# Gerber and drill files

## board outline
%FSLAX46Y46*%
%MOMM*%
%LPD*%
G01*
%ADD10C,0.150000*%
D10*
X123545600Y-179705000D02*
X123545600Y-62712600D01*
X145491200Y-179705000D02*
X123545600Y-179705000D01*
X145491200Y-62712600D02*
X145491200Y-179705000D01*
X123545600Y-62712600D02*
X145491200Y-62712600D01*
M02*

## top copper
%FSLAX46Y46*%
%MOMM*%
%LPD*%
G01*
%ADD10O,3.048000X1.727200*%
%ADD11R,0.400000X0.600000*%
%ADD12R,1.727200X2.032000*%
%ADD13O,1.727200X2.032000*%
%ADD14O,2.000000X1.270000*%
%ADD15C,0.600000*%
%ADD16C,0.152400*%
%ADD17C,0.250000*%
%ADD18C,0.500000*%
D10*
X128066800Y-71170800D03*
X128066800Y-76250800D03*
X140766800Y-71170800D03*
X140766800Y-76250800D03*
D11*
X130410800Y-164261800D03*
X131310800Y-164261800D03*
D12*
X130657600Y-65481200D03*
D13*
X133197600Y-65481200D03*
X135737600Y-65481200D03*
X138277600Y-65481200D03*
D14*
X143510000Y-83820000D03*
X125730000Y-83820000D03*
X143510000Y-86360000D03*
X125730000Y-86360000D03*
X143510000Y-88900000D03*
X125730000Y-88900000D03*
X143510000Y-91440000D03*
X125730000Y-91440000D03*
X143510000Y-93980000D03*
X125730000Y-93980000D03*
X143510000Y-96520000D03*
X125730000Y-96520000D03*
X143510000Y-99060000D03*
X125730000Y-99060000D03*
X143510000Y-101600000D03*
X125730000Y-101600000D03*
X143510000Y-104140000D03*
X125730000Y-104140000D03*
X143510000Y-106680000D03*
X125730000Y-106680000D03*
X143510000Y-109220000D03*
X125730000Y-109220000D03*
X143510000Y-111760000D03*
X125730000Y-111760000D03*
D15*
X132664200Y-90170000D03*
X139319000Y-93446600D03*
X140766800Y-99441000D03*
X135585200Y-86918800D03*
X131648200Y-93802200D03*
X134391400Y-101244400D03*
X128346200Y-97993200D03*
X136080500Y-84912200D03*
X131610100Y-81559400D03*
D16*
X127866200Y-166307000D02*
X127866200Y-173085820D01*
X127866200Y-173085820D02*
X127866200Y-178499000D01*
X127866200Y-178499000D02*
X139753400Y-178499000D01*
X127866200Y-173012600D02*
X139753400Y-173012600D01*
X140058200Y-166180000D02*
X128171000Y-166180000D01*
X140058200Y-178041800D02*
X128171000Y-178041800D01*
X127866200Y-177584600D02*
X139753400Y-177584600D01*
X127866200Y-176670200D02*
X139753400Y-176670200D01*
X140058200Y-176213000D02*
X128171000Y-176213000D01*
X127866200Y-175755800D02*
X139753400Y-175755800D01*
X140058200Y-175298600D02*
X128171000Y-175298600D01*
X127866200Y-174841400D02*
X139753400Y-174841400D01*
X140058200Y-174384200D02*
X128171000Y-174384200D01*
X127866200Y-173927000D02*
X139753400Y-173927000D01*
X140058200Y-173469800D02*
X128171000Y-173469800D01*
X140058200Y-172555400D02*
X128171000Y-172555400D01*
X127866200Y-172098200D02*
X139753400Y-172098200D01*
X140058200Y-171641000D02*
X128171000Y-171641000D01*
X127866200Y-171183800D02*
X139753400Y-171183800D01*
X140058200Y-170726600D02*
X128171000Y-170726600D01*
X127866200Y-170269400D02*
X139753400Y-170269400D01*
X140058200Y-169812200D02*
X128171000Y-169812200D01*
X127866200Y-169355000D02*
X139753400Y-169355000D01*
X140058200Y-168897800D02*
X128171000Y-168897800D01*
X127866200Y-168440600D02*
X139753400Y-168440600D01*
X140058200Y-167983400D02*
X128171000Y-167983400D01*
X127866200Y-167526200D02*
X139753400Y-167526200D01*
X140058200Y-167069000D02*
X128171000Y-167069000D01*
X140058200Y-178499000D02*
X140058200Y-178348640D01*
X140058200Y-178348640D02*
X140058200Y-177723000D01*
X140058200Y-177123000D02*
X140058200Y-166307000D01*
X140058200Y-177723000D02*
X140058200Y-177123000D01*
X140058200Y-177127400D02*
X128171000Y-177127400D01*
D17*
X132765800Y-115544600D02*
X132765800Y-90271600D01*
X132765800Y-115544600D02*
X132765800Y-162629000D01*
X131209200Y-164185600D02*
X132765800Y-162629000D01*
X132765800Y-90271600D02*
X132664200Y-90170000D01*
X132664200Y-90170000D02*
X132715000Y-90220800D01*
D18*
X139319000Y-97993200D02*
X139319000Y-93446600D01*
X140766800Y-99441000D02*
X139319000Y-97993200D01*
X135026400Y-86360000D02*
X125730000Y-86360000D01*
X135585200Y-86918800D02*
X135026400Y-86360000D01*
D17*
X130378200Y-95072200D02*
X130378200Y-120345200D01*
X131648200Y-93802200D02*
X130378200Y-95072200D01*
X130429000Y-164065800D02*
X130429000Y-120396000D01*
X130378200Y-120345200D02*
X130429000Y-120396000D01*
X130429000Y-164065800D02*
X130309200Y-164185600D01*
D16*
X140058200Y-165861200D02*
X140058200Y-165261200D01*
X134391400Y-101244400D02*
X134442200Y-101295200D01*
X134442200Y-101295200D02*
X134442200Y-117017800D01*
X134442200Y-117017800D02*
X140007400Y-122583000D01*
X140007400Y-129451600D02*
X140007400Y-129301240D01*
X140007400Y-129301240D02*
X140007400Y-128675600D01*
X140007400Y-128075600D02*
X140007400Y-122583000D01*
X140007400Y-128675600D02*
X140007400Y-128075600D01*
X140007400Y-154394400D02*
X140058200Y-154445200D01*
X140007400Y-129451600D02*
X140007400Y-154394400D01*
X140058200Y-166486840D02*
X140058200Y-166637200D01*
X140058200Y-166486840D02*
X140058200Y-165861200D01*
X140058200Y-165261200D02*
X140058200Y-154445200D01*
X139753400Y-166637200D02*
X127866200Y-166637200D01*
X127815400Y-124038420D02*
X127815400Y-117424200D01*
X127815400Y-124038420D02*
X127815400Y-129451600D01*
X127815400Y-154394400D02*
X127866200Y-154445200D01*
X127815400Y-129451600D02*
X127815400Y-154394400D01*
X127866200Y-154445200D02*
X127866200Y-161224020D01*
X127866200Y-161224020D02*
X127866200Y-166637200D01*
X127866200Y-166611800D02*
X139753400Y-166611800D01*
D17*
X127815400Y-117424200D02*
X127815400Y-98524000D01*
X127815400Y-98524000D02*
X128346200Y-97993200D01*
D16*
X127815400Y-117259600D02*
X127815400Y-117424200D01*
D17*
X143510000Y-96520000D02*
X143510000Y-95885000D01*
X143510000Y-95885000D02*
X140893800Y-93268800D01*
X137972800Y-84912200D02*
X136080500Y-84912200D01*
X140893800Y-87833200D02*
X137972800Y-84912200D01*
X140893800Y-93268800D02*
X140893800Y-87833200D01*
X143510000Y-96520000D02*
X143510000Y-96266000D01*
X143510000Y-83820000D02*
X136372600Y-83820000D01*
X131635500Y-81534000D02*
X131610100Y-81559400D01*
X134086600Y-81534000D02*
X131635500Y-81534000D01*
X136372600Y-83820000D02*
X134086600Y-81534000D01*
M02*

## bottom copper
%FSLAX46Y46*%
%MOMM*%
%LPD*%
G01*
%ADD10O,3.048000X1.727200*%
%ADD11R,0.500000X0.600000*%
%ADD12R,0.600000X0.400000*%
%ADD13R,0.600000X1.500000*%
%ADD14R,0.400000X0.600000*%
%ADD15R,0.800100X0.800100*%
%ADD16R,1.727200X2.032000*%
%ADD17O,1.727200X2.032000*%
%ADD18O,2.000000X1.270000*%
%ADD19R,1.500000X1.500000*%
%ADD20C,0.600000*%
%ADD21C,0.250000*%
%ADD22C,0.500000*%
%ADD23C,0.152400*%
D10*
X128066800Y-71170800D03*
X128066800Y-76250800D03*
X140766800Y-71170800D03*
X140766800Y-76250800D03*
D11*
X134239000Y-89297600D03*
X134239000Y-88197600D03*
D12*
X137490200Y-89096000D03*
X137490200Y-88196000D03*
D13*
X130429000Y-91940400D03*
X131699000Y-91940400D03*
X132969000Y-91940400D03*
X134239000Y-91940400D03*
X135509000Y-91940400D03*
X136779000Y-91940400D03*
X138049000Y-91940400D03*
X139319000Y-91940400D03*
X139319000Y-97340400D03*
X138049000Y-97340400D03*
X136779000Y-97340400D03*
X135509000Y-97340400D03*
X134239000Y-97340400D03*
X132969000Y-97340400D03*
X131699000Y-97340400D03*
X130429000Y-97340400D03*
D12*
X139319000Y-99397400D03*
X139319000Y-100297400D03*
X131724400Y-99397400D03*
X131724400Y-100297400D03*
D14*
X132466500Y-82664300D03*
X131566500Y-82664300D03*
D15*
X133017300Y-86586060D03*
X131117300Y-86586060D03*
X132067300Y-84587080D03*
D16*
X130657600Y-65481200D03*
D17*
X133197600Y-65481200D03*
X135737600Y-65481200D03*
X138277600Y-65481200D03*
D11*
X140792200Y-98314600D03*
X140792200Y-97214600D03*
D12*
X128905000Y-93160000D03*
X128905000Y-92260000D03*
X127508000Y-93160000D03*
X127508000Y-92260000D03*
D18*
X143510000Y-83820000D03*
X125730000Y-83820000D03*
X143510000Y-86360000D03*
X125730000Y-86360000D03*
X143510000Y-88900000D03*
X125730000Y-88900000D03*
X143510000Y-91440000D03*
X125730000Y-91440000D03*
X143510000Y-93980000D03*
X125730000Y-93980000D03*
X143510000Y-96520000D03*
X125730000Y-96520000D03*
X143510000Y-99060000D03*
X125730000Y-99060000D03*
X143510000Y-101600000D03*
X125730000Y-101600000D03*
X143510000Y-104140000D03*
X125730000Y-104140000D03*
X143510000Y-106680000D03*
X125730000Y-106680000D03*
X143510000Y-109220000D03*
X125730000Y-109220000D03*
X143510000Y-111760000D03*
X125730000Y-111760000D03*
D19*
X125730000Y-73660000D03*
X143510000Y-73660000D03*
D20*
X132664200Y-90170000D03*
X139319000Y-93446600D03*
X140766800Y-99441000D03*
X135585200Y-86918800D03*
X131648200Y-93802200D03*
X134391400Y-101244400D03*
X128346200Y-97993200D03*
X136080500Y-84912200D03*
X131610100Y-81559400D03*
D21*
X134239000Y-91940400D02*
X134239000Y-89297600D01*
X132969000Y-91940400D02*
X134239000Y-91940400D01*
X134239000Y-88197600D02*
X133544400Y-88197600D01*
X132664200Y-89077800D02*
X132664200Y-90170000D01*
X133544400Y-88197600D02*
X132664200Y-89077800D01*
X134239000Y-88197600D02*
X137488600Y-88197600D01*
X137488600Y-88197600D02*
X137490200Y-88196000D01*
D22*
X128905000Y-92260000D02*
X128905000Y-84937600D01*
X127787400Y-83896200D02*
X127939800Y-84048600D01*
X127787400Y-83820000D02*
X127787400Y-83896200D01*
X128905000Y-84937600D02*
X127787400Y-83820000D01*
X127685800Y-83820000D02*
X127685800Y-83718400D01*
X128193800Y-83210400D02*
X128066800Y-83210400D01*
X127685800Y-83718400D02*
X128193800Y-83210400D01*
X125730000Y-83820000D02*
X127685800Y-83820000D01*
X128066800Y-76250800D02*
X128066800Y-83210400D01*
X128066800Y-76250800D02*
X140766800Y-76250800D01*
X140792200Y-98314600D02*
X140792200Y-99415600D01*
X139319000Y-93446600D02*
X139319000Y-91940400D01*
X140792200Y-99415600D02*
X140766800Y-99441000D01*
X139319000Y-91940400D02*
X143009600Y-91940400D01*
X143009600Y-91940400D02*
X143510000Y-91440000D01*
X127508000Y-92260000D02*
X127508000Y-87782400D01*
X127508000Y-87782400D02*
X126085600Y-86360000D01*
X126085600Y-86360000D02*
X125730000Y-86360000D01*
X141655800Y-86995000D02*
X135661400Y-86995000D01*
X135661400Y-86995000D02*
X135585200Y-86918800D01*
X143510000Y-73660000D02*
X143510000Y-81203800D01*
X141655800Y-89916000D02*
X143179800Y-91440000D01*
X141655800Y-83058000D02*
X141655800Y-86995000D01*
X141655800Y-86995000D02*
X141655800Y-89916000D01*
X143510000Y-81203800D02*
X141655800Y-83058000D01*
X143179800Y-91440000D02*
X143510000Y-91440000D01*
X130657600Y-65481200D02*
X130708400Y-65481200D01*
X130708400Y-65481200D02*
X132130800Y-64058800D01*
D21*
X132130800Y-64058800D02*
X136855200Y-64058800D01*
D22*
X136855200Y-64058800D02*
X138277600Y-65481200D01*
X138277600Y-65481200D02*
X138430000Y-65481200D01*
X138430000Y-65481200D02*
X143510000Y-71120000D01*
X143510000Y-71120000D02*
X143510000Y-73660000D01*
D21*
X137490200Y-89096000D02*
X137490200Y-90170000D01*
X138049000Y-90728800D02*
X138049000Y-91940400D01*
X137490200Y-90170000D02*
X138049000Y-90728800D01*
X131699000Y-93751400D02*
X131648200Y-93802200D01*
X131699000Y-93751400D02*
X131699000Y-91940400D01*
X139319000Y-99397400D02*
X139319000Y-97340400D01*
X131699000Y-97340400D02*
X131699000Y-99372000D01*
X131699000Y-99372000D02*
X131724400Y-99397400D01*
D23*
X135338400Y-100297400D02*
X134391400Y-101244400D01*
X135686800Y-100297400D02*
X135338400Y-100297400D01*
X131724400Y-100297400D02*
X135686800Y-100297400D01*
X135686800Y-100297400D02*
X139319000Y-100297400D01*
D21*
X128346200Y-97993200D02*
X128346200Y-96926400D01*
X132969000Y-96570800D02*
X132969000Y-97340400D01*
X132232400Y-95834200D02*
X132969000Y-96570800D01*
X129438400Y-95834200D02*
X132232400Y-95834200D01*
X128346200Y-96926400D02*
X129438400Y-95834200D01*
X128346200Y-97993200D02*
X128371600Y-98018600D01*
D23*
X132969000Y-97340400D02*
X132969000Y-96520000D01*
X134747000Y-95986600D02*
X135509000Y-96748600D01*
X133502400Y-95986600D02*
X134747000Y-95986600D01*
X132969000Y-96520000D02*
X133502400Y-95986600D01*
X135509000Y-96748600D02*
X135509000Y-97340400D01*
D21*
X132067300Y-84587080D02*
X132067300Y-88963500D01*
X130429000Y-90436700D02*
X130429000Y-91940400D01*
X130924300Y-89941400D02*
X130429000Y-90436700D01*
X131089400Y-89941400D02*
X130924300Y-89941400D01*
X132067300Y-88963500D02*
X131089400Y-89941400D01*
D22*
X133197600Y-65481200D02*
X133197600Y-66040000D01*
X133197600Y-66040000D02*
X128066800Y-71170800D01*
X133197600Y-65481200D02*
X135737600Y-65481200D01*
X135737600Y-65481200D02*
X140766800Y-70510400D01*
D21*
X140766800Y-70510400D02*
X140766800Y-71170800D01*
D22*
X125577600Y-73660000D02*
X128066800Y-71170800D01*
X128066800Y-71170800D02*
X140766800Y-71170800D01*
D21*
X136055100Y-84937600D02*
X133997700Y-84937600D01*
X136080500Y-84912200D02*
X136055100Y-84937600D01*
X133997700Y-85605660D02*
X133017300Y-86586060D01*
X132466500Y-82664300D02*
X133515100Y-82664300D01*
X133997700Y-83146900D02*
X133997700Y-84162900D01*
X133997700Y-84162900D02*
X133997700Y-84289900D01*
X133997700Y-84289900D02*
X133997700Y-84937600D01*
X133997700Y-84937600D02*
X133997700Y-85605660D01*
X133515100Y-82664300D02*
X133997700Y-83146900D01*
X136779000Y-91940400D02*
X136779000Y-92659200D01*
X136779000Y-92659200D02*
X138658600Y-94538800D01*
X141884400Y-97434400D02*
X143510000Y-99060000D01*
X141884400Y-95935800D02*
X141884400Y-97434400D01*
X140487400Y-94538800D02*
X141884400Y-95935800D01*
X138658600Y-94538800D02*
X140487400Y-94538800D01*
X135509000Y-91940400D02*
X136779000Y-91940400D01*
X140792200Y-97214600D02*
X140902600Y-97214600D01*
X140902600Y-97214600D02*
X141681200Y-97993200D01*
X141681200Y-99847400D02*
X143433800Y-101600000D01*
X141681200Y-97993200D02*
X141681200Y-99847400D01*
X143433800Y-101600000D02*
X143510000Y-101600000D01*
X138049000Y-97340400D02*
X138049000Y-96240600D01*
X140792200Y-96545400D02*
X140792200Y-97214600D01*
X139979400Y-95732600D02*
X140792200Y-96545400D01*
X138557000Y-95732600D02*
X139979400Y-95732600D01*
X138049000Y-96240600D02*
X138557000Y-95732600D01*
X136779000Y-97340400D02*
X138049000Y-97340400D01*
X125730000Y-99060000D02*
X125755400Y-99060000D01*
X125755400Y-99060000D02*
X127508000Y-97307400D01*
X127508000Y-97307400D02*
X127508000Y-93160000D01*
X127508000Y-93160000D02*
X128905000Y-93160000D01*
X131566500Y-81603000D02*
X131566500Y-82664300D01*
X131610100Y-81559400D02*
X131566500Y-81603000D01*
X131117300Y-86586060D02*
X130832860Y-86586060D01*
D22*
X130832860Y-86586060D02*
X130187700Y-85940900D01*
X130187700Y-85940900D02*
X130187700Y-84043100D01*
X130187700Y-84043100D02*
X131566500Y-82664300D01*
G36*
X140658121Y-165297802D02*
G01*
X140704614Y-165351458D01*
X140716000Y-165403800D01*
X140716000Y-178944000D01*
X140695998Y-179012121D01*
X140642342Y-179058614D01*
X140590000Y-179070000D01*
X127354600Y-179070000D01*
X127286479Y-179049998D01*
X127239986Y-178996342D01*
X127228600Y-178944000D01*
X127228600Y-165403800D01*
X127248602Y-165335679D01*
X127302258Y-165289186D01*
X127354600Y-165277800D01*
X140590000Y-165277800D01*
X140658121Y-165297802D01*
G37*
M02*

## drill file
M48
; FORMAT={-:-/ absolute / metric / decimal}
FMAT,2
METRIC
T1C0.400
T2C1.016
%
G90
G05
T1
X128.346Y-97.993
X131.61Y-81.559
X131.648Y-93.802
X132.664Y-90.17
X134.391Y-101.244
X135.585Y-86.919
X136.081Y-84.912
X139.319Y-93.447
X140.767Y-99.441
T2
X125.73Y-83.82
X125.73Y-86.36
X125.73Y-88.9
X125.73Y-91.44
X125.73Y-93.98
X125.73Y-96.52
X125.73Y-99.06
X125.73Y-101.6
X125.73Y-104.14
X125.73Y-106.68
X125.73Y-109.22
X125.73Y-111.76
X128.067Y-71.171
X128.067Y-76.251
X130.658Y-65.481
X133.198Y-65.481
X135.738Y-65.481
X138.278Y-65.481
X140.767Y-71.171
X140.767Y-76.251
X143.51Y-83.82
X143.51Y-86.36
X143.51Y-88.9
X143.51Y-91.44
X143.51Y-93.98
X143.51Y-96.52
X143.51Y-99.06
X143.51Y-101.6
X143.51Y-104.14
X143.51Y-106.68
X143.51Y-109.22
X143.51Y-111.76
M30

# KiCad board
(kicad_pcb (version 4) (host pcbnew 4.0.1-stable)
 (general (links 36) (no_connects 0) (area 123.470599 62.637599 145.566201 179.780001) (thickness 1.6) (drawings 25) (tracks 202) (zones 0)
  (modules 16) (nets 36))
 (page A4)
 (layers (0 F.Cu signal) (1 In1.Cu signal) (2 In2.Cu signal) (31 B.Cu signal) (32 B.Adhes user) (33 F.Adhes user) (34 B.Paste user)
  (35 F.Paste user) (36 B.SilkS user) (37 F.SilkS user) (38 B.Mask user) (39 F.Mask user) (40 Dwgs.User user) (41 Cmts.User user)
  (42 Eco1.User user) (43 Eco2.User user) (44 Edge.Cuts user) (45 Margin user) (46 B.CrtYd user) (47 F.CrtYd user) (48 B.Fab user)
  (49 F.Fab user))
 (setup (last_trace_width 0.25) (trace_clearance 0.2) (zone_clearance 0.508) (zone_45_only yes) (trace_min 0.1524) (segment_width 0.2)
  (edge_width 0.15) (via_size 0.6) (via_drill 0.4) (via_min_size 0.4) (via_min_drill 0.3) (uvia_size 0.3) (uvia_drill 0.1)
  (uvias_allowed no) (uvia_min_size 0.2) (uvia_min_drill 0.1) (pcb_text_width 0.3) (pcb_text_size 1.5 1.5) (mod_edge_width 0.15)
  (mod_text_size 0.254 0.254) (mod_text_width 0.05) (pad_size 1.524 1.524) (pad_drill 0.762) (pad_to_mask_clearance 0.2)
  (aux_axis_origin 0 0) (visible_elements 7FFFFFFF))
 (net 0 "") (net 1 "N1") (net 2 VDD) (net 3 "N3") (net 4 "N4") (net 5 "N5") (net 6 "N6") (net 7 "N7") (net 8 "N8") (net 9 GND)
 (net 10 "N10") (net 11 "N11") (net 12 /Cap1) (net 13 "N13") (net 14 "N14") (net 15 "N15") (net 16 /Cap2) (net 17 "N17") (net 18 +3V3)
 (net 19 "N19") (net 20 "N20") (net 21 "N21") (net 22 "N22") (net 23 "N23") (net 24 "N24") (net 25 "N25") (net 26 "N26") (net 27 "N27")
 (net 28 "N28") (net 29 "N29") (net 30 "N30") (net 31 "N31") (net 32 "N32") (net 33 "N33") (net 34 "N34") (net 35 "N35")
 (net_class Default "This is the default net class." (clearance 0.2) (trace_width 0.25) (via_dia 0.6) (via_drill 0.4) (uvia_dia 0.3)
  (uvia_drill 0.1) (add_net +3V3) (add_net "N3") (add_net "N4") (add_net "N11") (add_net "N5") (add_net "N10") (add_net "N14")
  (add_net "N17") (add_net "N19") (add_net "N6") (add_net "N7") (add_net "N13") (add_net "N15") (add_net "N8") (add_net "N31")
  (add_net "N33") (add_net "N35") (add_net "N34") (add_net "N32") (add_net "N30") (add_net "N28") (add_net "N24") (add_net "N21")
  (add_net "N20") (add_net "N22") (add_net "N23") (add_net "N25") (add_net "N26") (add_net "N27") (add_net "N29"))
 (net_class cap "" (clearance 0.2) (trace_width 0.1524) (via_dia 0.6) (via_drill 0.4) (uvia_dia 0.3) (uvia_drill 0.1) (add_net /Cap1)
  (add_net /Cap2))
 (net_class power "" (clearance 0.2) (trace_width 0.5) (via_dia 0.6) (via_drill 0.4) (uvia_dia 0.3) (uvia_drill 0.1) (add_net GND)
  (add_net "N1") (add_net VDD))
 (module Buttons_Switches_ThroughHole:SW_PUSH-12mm (layer B.Cu) (at 134.4168 73.7108 180)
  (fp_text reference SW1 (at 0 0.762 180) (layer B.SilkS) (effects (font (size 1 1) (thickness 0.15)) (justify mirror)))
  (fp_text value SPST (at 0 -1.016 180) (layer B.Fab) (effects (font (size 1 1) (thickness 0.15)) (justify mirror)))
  (pad 1 thru_hole oval (at 6.35 2.54 180) (size 3.048 1.7272) (drill 1.016) (layers *.Cu *.Mask B.SilkS) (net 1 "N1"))
  (pad 2 thru_hole oval (at 6.35 -2.54 180) (size 3.048 1.7272) (drill 1.016) (layers *.Cu *.Mask B.SilkS) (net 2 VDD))
  (pad 1 thru_hole oval (at -6.35 2.54 180) (size 3.048 1.7272) (drill 1.016) (layers *.Cu *.Mask B.SilkS) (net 1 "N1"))
  (pad 2 thru_hole oval (at -6.35 -2.54 180) (size 3.048 1.7272) (drill 1.016) (layers *.Cu *.Mask B.SilkS) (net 2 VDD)))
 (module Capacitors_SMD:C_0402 (layer B.Cu) (at 134.239 88.7476 90)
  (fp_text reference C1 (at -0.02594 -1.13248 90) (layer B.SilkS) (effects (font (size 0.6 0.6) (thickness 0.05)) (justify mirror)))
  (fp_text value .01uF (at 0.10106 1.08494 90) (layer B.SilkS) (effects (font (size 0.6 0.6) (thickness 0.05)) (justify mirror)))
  (pad 1 smd rect (at -0.55 0 90) (size 0.6 0.5) (layers B.Cu B.Paste B.Mask) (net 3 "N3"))
  (pad 2 smd rect (at 0.55 0 90) (size 0.6 0.5) (layers B.Cu B.Paste B.Mask) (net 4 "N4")))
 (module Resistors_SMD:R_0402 (layer B.Cu) (at 137.4902 88.646 90)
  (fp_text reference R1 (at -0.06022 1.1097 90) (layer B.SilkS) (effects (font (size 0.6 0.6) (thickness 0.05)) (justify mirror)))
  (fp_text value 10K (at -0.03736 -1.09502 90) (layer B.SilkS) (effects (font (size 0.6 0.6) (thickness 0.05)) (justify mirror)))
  (pad 1 smd rect (at -0.45 0 90) (size 0.4 0.6) (layers B.Cu B.Paste B.Mask) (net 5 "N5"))
  (pad 2 smd rect (at 0.45 0 90) (size 0.4 0.6) (layers B.Cu B.Paste B.Mask) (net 4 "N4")))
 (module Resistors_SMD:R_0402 (layer F.Cu) (at 130.8608 164.2618)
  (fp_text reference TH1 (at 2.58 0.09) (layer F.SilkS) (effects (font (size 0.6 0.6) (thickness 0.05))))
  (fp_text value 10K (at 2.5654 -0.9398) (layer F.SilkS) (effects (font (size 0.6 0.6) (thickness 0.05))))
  (pad 1 smd rect (at -0.45 0) (size 0.4 0.6) (layers F.Cu F.Paste F.Mask) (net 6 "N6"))
  (pad 2 smd rect (at 0.45 0) (size 0.4 0.6) (layers F.Cu F.Paste F.Mask) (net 4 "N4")))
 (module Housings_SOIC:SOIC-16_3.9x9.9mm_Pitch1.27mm (layer B.Cu) (at 134.874 94.6404 270)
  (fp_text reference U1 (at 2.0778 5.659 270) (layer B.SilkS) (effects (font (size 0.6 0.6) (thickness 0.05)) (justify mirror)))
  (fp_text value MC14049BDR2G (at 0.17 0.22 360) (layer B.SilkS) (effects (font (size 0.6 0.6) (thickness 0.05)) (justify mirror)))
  (pad 1 smd rect (at -2.7 4.445 270) (size 1.5 0.6) (layers B.Cu B.Paste B.Mask) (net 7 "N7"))
  (pad 2 smd rect (at -2.7 3.175 270) (size 1.5 0.6) (layers B.Cu B.Paste B.Mask) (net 6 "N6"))
  (pad 3 smd rect (at -2.7 1.905 270) (size 1.5 0.6) (layers B.Cu B.Paste B.Mask) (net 3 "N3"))
  (pad 4 smd rect (at -2.7 0.635 270) (size 1.5 0.6) (layers B.Cu B.Paste B.Mask) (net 3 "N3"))
  (pad 5 smd rect (at -2.7 -0.635 270) (size 1.5 0.6) (layers B.Cu B.Paste B.Mask) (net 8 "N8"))
  (pad 6 smd rect (at -2.7 -1.905 270) (size 1.5 0.6) (layers B.Cu B.Paste B.Mask) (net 8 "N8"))
  (pad 7 smd rect (at -2.7 -3.175 270) (size 1.5 0.6) (layers B.Cu B.Paste B.Mask) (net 5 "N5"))
  (pad 8 smd rect (at -2.7 -4.445 270) (size 1.5 0.6) (layers B.Cu B.Paste B.Mask) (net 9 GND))
  (pad 9 smd rect (at 2.7 -4.445 270) (size 1.5 0.6) (layers B.Cu B.Paste B.Mask) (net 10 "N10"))
  (pad 10 smd rect (at 2.7 -3.175 270) (size 1.5 0.6) (layers B.Cu B.Paste B.Mask) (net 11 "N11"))
  (pad 11 smd rect (at 2.7 -1.905 270) (size 1.5 0.6) (layers B.Cu B.Paste B.Mask) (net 11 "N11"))
  (pad 12 smd rect (at 2.7 -0.635 270) (size 1.5 0.6) (layers B.Cu B.Paste B.Mask) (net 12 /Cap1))
  (pad 13 smd rect (at 2.7 0.635 270) (size 1.5 0.6) (layers B.Cu B.Paste B.Mask) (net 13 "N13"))
  (pad 14 smd rect (at 2.7 1.905 270) (size 1.5 0.6) (layers B.Cu B.Paste B.Mask) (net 12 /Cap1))
  (pad 15 smd rect (at 2.7 3.175 270) (size 1.5 0.6) (layers B.Cu B.Paste B.Mask) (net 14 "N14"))
  (pad 16 smd rect (at 2.7 4.445 270) (size 1.5 0.6) (layers B.Cu B.Paste B.Mask) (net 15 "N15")))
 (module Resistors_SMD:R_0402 (layer B.Cu) (at 139.319 99.8474 270)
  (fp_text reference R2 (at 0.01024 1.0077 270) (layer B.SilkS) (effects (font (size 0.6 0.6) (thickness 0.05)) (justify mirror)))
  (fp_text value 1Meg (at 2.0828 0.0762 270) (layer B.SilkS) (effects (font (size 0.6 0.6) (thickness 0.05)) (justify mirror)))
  (pad 1 smd rect (at -0.45 0 270) (size 0.4 0.6) (layers B.Cu B.Paste B.Mask) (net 10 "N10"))
  (pad 2 smd rect (at 0.45 0 270) (size 0.4 0.6) (layers B.Cu B.Paste B.Mask) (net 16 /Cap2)))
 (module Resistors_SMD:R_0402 (layer B.Cu) (at 131.7244 99.8474 270)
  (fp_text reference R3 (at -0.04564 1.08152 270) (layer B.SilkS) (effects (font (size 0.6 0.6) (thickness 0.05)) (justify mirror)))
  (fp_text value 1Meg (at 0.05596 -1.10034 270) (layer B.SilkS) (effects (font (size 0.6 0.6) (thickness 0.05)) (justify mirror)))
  (pad 1 smd rect (at -0.45 0 270) (size 0.4 0.6) (layers B.Cu B.Paste B.Mask) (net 14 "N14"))
  (pad 2 smd rect (at 0.45 0 270) (size 0.4 0.6) (layers B.Cu B.Paste B.Mask) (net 16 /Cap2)))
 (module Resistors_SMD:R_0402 (layer B.Cu) (at 132.0165 82.6643 180)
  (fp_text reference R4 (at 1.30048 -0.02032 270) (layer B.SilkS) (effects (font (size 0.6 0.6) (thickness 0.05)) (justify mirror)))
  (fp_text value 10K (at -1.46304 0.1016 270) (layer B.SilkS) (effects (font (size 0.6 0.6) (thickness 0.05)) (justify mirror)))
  (pad 1 smd rect (at -0.45 0 180) (size 0.4 0.6) (layers B.Cu B.Paste B.Mask) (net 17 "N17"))
  (pad 2 smd rect (at 0.45 0 180) (size 0.4 0.6) (layers B.Cu B.Paste B.Mask) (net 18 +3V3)))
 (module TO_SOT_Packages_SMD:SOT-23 (layer B.Cu) (at 132.0673 85.5853 180)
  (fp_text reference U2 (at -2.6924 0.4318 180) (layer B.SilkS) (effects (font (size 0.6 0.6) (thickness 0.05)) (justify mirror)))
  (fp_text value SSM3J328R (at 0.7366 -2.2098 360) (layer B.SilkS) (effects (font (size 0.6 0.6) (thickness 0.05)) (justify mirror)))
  (pad 1 smd rect (at -0.95 -1.00076 180) (size 0.8001 0.8001) (layers B.Cu B.Paste B.Mask) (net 17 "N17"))
  (pad 2 smd rect (at 0.95 -1.00076 180) (size 0.8001 0.8001) (layers B.Cu B.Paste B.Mask) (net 18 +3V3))
  (pad 3 smd rect (at 0 0.99822 180) (size 0.8001 0.8001) (layers B.Cu B.Paste B.Mask) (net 7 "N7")))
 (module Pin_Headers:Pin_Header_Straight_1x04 (layer F.Cu) (at 130.6576 65.4812 90)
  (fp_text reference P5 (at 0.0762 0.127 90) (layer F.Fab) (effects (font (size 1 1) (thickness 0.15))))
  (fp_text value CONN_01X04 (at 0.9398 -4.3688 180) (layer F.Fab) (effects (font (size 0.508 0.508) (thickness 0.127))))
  (pad 1 thru_hole rect (at 0 0 90) (size 2.032 1.7272) (drill 1.016) (layers *.Cu *.Mask F.SilkS) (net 9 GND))
  (pad 2 thru_hole oval (at 0 2.54 90) (size 2.032 1.7272) (drill 1.016) (layers *.Cu *.Mask F.SilkS) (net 1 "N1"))
  (pad 3 thru_hole oval (at 0 5.08 90) (size 2.032 1.7272) (drill 1.016) (layers *.Cu *.Mask F.SilkS) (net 1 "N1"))
  (pad 4 thru_hole oval (at 0 7.62 90) (size 2.032 1.7272) (drill 1.016) (layers *.Cu *.Mask F.SilkS) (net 9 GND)))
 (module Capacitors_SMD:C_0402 (layer B.Cu) (at 140.7922 97.7646 90)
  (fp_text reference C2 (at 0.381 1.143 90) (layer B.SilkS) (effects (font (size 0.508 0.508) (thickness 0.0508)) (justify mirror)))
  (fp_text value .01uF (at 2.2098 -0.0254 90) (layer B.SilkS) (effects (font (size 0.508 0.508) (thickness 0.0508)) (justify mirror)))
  (pad 1 smd rect (at -0.55 0 90) (size 0.6 0.5) (layers B.Cu B.Paste B.Mask) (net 9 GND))
  (pad 2 smd rect (at 0.55 0 90) (size 0.6 0.5) (layers B.Cu B.Paste B.Mask) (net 11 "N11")))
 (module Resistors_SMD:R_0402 (layer B.Cu) (at 128.905 92.71 90)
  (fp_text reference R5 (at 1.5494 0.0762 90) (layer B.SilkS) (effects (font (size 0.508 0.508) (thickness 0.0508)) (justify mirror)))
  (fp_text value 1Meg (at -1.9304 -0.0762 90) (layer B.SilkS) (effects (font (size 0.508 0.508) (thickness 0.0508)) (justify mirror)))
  (pad 1 smd rect (at -0.45 0 90) (size 0.4 0.6) (layers B.Cu B.Paste B.Mask) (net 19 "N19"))
  (pad 2 smd rect (at 0.45 0 90) (size 0.4 0.6) (layers B.Cu B.Paste B.Mask) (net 2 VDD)))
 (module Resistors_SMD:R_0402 (layer B.Cu) (at 127.508 92.71 90)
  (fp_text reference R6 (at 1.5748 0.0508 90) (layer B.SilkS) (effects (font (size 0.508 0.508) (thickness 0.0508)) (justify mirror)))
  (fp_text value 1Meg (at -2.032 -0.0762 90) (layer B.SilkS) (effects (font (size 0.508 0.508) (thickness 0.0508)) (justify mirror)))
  (pad 1 smd rect (at -0.45 0 90) (size 0.4 0.6) (layers B.Cu B.Paste B.Mask) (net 19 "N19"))
  (pad 2 smd rect (at 0.45 0 90) (size 0.4 0.6) (layers B.Cu B.Paste B.Mask) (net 9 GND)))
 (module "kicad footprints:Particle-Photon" (layer F.Cu) (at 134.62 97.79 270)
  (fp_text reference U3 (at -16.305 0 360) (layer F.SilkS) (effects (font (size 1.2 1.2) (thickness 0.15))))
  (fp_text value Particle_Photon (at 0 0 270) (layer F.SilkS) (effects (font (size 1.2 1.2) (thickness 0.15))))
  (pad 24 thru_hole oval (at -13.97 -8.89 270) (size 1.27 2) (drill 1.016) (layers *.Cu *.Mask F.SilkS) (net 18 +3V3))
  (pad 1 thru_hole oval (at -13.97 8.89 270) (size 1.27 2) (drill 1.016) (layers *.Cu *.Mask F.SilkS) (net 2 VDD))
  (pad 23 thru_hole oval (at -11.43 -8.89 270) (size 1.27 2) (drill 1.016) (layers *.Cu *.Mask F.SilkS) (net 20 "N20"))
  (pad 2 thru_hole oval (at -11.43 8.89 270) (size 1.27 2) (drill 1.016) (layers *.Cu *.Mask F.SilkS) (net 9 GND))
  (pad 22 thru_hole oval (at -8.89 -8.89 270) (size 1.27 2) (drill 1.016) (layers *.Cu *.Mask F.SilkS) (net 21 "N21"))
  (pad 3 thru_hole oval (at -8.89 8.89 270) (size 1.27 2) (drill 1.016) (layers *.Cu *.Mask F.SilkS) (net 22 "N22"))
  (pad 21 thru_hole oval (at -6.35 -8.89 270) (size 1.27 2) (drill 1.016) (layers *.Cu *.Mask F.SilkS) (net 9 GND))
  (pad 4 thru_hole oval (at -6.35 8.89 270) (size 1.27 2) (drill 1.016) (layers *.Cu *.Mask F.SilkS) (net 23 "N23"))
  (pad 20 thru_hole oval (at -3.81 -8.89 270) (size 1.27 2) (drill 1.016) (layers *.Cu *.Mask F.SilkS) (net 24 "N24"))
  (pad 5 thru_hole oval (at -3.81 8.89 270) (size 1.27 2) (drill 1.016) (layers *.Cu *.Mask F.SilkS) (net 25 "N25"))
  (pad 19 thru_hole oval (at -1.27 -8.89 270) (size 1.27 2) (drill 1.016) (layers *.Cu *.Mask F.SilkS) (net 17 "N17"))
  (pad 6 thru_hole oval (at -1.27 8.89 270) (size 1.27 2) (drill 1.016) (layers *.Cu *.Mask F.SilkS) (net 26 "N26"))
  (pad 18 thru_hole oval (at 1.27 -8.89 270) (size 1.27 2) (drill 1.016) (layers *.Cu *.Mask F.SilkS) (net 8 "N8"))
  (pad 7 thru_hole oval (at 1.27 8.89 270) (size 1.27 2) (drill 1.016) (layers *.Cu *.Mask F.SilkS) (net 19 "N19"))
  (pad 17 thru_hole oval (at 3.81 -8.89 270) (size 1.27 2) (drill 1.016) (layers *.Cu *.Mask F.SilkS) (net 11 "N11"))
  (pad 8 thru_hole oval (at 3.81 8.89 270) (size 1.27 2) (drill 1.016) (layers *.Cu *.Mask F.SilkS) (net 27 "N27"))
  (pad 16 thru_hole oval (at 6.35 -8.89 270) (size 1.27 2) (drill 1.016) (layers *.Cu *.Mask F.SilkS) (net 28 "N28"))
  (pad 9 thru_hole oval (at 6.35 8.89 270) (size 1.27 2) (drill 1.016) (layers *.Cu *.Mask F.SilkS) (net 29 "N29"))
  (pad 15 thru_hole oval (at 8.89 -8.89 270) (size 1.27 2) (drill 1.016) (layers *.Cu *.Mask F.SilkS) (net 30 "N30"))
  (pad 10 thru_hole oval (at 8.89 8.89 270) (size 1.27 2) (drill 1.016) (layers *.Cu *.Mask F.SilkS) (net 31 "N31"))
  (pad 14 thru_hole oval (at 11.43 -8.89 270) (size 1.27 2) (drill 1.016) (layers *.Cu *.Mask F.SilkS) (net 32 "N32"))
  (pad 11 thru_hole oval (at 11.43 8.89 270) (size 1.27 2) (drill 1.016) (layers *.Cu *.Mask F.SilkS) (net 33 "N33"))
  (pad 13 thru_hole oval (at 13.97 -8.89 270) (size 1.27 2) (drill 1.016) (layers *.Cu *.Mask F.SilkS) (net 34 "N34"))
  (pad 12 thru_hole oval (at 13.97 8.89 270) (size 1.27 2) (drill 1.016) (layers *.Cu *.Mask F.SilkS) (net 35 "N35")))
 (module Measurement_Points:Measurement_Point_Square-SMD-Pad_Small (layer B.Cu) (at 125.73 73.66)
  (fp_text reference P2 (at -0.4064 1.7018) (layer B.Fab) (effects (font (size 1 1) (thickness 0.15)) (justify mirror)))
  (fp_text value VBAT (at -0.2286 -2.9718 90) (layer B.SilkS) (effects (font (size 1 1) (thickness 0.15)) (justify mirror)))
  (pad 1 smd rect (at 0 0) (size 1.5 1.5) (layers B.Cu B.Mask) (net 1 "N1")))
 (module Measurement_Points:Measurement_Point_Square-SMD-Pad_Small (layer B.Cu) (at 143.51 73.66)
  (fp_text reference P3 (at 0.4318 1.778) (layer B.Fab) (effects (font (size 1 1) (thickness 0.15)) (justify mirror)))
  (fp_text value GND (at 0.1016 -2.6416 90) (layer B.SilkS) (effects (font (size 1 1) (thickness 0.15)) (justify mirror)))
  (pad 1 smd rect (at 0 0) (size 1.5 1.5) (layers B.Cu B.Mask) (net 9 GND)))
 (gr_line (start 123.5456 179.705) (end 123.5456 62.7126) (angle 90) (layer Edge.Cuts) (width 0.15))
 (gr_line (start 145.4912 179.705) (end 123.5456 179.705) (angle 90) (layer Edge.Cuts) (width 0.15))
 (gr_line (start 145.4912 62.7126) (end 145.4912 179.705) (angle 90) (layer Edge.Cuts) (width 0.15))
 (gr_line (start 123.5456 62.7126) (end 145.4912 62.7126) (angle 90) (layer Edge.Cuts) (width 0.15))
 (segment (start 127.8662 166.307) (end 127.8662 173.08582) (width 0.1524) (layer F.Cu) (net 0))
 (segment (start 127.8662 173.08582) (end 127.8662 178.499) (width 0.1524) (layer F.Cu) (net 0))
 (segment (start 127.8662 178.499) (end 139.7534 178.499) (width 0.1524) (layer F.Cu) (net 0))
 (segment (start 127.8662 173.0126) (end 139.7534 173.0126) (width 0.1524) (layer F.Cu) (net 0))
 (segment (start 140.0582 166.18) (end 128.171 166.18) (width 0.1524) (layer F.Cu) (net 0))
 (segment (start 140.0582 178.0418) (end 128.171 178.0418) (width 0.1524) (layer F.Cu) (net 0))
 (segment (start 127.8662 177.5846) (end 139.7534 177.5846) (width 0.1524) (layer F.Cu) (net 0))
 (segment (start 127.8662 176.6702) (end 139.7534 176.6702) (width 0.1524) (layer F.Cu) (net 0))
 (segment (start 140.0582 176.213) (end 128.171 176.213) (width 0.1524) (layer F.Cu) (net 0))
 (segment (start 127.8662 175.7558) (end 139.7534 175.7558) (width 0.1524) (layer F.Cu) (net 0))
 (segment (start 140.0582 175.2986) (end 128.171 175.2986) (width 0.1524) (layer F.Cu) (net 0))
 (segment (start 127.8662 174.8414) (end 139.7534 174.8414) (width 0.1524) (layer F.Cu) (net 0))
 (segment (start 140.0582 174.3842) (end 128.171 174.3842) (width 0.1524) (layer F.Cu) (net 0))
 (segment (start 127.8662 173.927) (end 139.7534 173.927) (width 0.1524) (layer F.Cu) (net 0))
 (segment (start 140.0582 173.4698) (end 128.171 173.4698) (width 0.1524) (layer F.Cu) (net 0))
 (segment (start 140.0582 172.5554) (end 128.171 172.5554) (width 0.1524) (layer F.Cu) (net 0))
 (segment (start 127.8662 172.0982) (end 139.7534 172.0982) (width 0.1524) (layer F.Cu) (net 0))
 (segment (start 140.0582 171.641) (end 128.171 171.641) (width 0.1524) (layer F.Cu) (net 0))
 (segment (start 127.8662 171.1838) (end 139.7534 171.1838) (width 0.1524) (layer F.Cu) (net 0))
 (segment (start 140.0582 170.7266) (end 128.171 170.7266) (width 0.1524) (layer F.Cu) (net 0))
 (segment (start 127.8662 170.2694) (end 139.7534 170.2694) (width 0.1524) (layer F.Cu) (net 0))
 (segment (start 140.0582 169.8122) (end 128.171 169.8122) (width 0.1524) (layer F.Cu) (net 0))
 (segment (start 127.8662 169.355) (end 139.7534 169.355) (width 0.1524) (layer F.Cu) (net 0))
 (segment (start 140.0582 168.8978) (end 128.171 168.8978) (width 0.1524) (layer F.Cu) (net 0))
 (segment (start 127.8662 168.4406) (end 139.7534 168.4406) (width 0.1524) (layer F.Cu) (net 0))
 (segment (start 140.0582 167.9834) (end 128.171 167.9834) (width 0.1524) (layer F.Cu) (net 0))
 (segment (start 127.8662 167.5262) (end 139.7534 167.5262) (width 0.1524) (layer F.Cu) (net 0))
 (segment (start 140.0582 167.069) (end 128.171 167.069) (width 0.1524) (layer F.Cu) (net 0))
 (segment (start 140.0582 178.499) (end 140.0582 178.34864) (width 0.1524) (layer F.Cu) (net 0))
 (segment (start 140.0582 178.34864) (end 140.0582 177.723) (width 0.1524) (layer F.Cu) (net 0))
 (segment (start 140.0582 177.123) (end 140.0582 166.307) (width 0.1524) (layer F.Cu) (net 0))
 (segment (start 140.0582 177.723) (end 140.0582 177.123) (width 0.1524) (layer F.Cu) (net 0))
 (segment (start 140.0582 177.1274) (end 128.171 177.1274) (width 0.1524) (layer F.Cu) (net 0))
 (segment (start 134.239 91.9404) (end 134.239 89.2976) (width 0.25) (layer B.Cu) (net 3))
 (segment (start 132.969 91.9404) (end 134.239 91.9404) (width 0.25) (layer B.Cu) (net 3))
 (segment (start 132.7658 115.5446) (end 132.7658 90.2716) (width 0.25) (layer F.Cu) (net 4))
 (segment (start 132.7658 115.5446) (end 132.7658 162.629) (width 0.25) (layer F.Cu) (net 4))
 (segment (start 131.2092 164.1856) (end 132.7658 162.629) (width 0.25) (layer F.Cu) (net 4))
 (segment (start 132.7658 90.2716) (end 132.6642 90.17) (width 0.25) (layer F.Cu) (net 4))
 (segment (start 134.239 88.1976) (end 133.5444 88.1976) (width 0.25) (layer B.Cu) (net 4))
 (segment (start 132.6642 90.17) (end 132.715 90.2208) (width 0.25) (layer F.Cu) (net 4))
 (via (at 132.6642 90.17) (size 0.6) (drill 0.4) (layers F.Cu B.Cu) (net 4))
 (segment (start 132.6642 89.0778) (end 132.6642 90.17) (width 0.25) (layer B.Cu) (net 4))
 (segment (start 133.5444 88.1976) (end 132.6642 89.0778) (width 0.25) (layer B.Cu) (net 4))
 (segment (start 134.239 88.1976) (end 137.4886 88.1976) (width 0.25) (layer B.Cu) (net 4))
 (segment (start 137.4886 88.1976) (end 137.4902 88.196) (width 0.25) (layer B.Cu) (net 4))
 (segment (start 128.905 92.26) (end 128.905 84.9376) (width 0.5) (layer B.Cu) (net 2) (status 400000))
 (segment (start 127.7874 83.8962) (end 127.9398 84.0486) (width 0.5) (layer B.Cu) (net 2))
 (segment (start 127.7874 83.82) (end 127.7874 83.8962) (width 0.5) (layer B.Cu) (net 2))
 (segment (start 128.905 84.9376) (end 127.7874 83.82) (width 0.5) (layer B.Cu) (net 2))
 (segment (start 127.6858 83.82) (end 127.6858 83.7184) (width 0.5) (layer B.Cu) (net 2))
 (segment (start 128.1938 83.2104) (end 128.0668 83.2104) (width 0.5) (layer B.Cu) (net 2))
 (segment (start 127.6858 83.7184) (end 128.1938 83.2104) (width 0.5) (layer B.Cu) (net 2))
 (segment (start 125.73 83.82) (end 127.6858 83.82) (width 0.5) (layer B.Cu) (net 2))
 (segment (start 128.0668 76.2508) (end 128.0668 83.2104) (width 0.5) (layer B.Cu) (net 2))
 (segment (start 128.0668 76.2508) (end 140.7668 76.2508) (width 0.5) (layer B.Cu) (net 2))
 (segment (start 140.7922 98.3146) (end 140.7922 99.4156) (width 0.5) (layer B.Cu) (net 9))
 (segment (start 139.319 93.4466) (end 139.319 91.9404) (width 0.5) (layer B.Cu) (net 9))
 (via (at 139.319 93.4466) (size 0.6) (drill 0.4) (layers F.Cu B.Cu) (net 9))
 (segment (start 139.319 97.9932) (end 139.319 93.4466) (width 0.5) (layer F.Cu) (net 9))
 (segment (start 140.7668 99.441) (end 139.319 97.9932) (width 0.5) (layer F.Cu) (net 9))
 (via (at 140.7668 99.441) (size 0.6) (drill 0.4) (layers F.Cu B.Cu) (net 9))
 (segment (start 140.7922 99.4156) (end 140.7668 99.441) (width 0.5) (layer B.Cu) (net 9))
 (segment (start 139.319 91.9404) (end 143.0096 91.9404) (width 0.5) (layer B.Cu) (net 9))
 (segment (start 143.0096 91.9404) (end 143.51 91.44) (width 0.5) (layer B.Cu) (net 9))
 (segment (start 127.508 92.26) (end 127.508 87.7824) (width 0.5) (layer B.Cu) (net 9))
 (segment (start 127.508 87.7824) (end 126.0856 86.36) (width 0.5) (layer B.Cu) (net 9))
 (segment (start 126.0856 86.36) (end 125.73 86.36) (width 0.5) (layer B.Cu) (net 9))
 (segment (start 141.6558 86.995) (end 135.6614 86.995) (width 0.5) (layer B.Cu) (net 9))
 (segment (start 135.0264 86.36) (end 125.73 86.36) (width 0.5) (layer F.Cu) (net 9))
 (segment (start 135.5852 86.9188) (end 135.0264 86.36) (width 0.5) (layer F.Cu) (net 9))
 (via (at 135.5852 86.9188) (size 0.6) (drill 0.4) (layers F.Cu B.Cu) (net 9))
 (segment (start 135.6614 86.995) (end 135.5852 86.9188) (width 0.5) (layer B.Cu) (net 9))
 (segment (start 143.51 73.66) (end 143.51 81.2038) (width 0.5) (layer B.Cu) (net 9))
 (segment (start 141.6558 89.916) (end 143.1798 91.44) (width 0.5) (layer B.Cu) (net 9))
 (segment (start 141.6558 83.058) (end 141.6558 86.995) (width 0.5) (layer B.Cu) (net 9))
 (segment (start 141.6558 86.995) (end 141.6558 89.916) (width 0.5) (layer B.Cu) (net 9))
 (segment (start 143.51 81.2038) (end 141.6558 83.058) (width 0.5) (layer B.Cu) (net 9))
 (segment (start 143.1798 91.44) (end 143.51 91.44) (width 0.5) (layer B.Cu) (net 9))
 (segment (start 130.6576 65.4812) (end 130.7084 65.4812) (width 0.5) (layer B.Cu) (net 9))
 (segment (start 130.7084 65.4812) (end 132.1308 64.0588) (width 0.5) (layer B.Cu) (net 9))
 (segment (start 132.1308 64.0588) (end 136.8552 64.0588) (width 0.25) (layer B.Cu) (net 9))
 (segment (start 136.8552 64.0588) (end 138.2776 65.4812) (width 0.5) (layer B.Cu) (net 9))
 (segment (start 138.2776 65.4812) (end 138.43 65.4812) (width 0.5) (layer B.Cu) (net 9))
 (segment (start 138.43 65.4812) (end 143.51 71.12) (width 0.5) (layer B.Cu) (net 9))
 (segment (start 143.51 71.12) (end 143.51 73.66) (width 0.5) (layer B.Cu) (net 9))
 (segment (start 137.4902 89.096) (end 137.4902 90.17) (width 0.25) (layer B.Cu) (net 5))
 (segment (start 138.049 90.7288) (end 138.049 91.9404) (width 0.25) (layer B.Cu) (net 5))
 (segment (start 137.4902 90.17) (end 138.049 90.7288) (width 0.25) (layer B.Cu) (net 5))
 (segment (start 130.3782 95.0722) (end 130.3782 120.3452) (width 0.25) (layer F.Cu) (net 6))
 (segment (start 131.699 93.7514) (end 131.6482 93.8022) (width 0.25) (layer B.Cu) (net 6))
 (via (at 131.6482 93.8022) (size 0.6) (drill 0.4) (layers F.Cu B.Cu) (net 6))
 (segment (start 131.6482 93.8022) (end 130.3782 95.0722) (width 0.25) (layer F.Cu) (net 6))
 (segment (start 130.429 164.0658) (end 130.429 120.396) (width 0.25) (layer F.Cu) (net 6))
 (segment (start 131.699 93.7514) (end 131.699 91.9404) (width 0.25) (layer B.Cu) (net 6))
 (segment (start 130.3782 120.3452) (end 130.429 120.396) (width 0.25) (layer F.Cu) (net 6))
 (segment (start 130.429 164.0658) (end 130.3092 164.1856) (width 0.25) (layer F.Cu) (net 6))
 (segment (start 139.319 99.3974) (end 139.319 97.3404) (width 0.25) (layer B.Cu) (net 10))
 (segment (start 131.699 97.3404) (end 131.699 99.372) (width 0.25) (layer B.Cu) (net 14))
 (segment (start 131.699 99.372) (end 131.7244 99.3974) (width 0.25) (layer B.Cu) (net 14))
 (segment (start 140.0582 165.8612) (end 140.0582 165.2612) (width 0.1524) (layer F.Cu) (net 16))
 (segment (start 135.3384 100.2974) (end 134.3914 101.2444) (width 0.1524) (layer B.Cu) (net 16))
 (via (at 134.3914 101.2444) (size 0.6) (drill 0.4) (layers F.Cu B.Cu) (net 16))
 (segment (start 134.3914 101.2444) (end 134.4422 101.2952) (width 0.1524) (layer F.Cu) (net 16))
 (segment (start 134.4422 101.2952) (end 134.4422 117.0178) (width 0.1524) (layer F.Cu) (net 16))
 (segment (start 134.4422 117.0178) (end 140.0074 122.583) (width 0.1524) (layer F.Cu) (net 16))
 (segment (start 135.6868 100.2974) (end 135.3384 100.2974) (width 0.1524) (layer B.Cu) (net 16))
 (segment (start 140.0074 129.4516) (end 140.0074 129.30124) (width 0.1524) (layer F.Cu) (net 16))
 (segment (start 140.0074 129.30124) (end 140.0074 128.6756) (width 0.1524) (layer F.Cu) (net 16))
 (segment (start 140.0074 128.0756) (end 140.0074 122.583) (width 0.1524) (layer F.Cu) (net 16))
 (segment (start 140.0074 128.6756) (end 140.0074 128.0756) (width 0.1524) (layer F.Cu) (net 16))
 (segment (start 140.0074 154.3944) (end 140.0582 154.4452) (width 0.1524) (layer F.Cu) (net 16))
 (segment (start 140.0074 129.4516) (end 140.0074 154.3944) (width 0.1524) (layer F.Cu) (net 16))
 (segment (start 140.0582 166.48684) (end 140.0582 166.6372) (width 0.1524) (layer F.Cu) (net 16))
 (segment (start 140.0582 166.48684) (end 140.0582 165.8612) (width 0.1524) (layer F.Cu) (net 16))
 (segment (start 140.0582 165.2612) (end 140.0582 154.4452) (width 0.1524) (layer F.Cu) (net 16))
 (segment (start 131.7244 100.2974) (end 135.6868 100.2974) (width 0.1524) (layer B.Cu) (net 16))
 (segment (start 135.6868 100.2974) (end 139.319 100.2974) (width 0.1524) (layer B.Cu) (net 16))
 (segment (start 139.7534 166.6372) (end 127.8662 166.6372) (width 0.1524) (layer F.Cu) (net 12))
 (segment (start 127.8154 124.03842) (end 127.8154 117.4242) (width 0.1524) (layer F.Cu) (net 12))
 (segment (start 127.8154 124.03842) (end 127.8154 129.4516) (width 0.1524) (layer F.Cu) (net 12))
 (segment (start 127.8154 154.3944) (end 127.8662 154.4452) (width 0.1524) (layer F.Cu) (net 12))
 (segment (start 127.8154 129.4516) (end 127.8154 154.3944) (width 0.1524) (layer F.Cu) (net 12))
 (segment (start 127.8662 154.4452) (end 127.8662 161.22402) (width 0.1524) (layer F.Cu) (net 12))
 (segment (start 127.8662 161.22402) (end 127.8662 166.6372) (width 0.1524) (layer F.Cu) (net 12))
 (segment (start 127.8662 166.6118) (end 139.7534 166.6118) (width 0.1524) (layer F.Cu) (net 12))
 (segment (start 128.3462 97.9932) (end 128.3462 96.9264) (width 0.25) (layer B.Cu) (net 12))
 (segment (start 132.969 96.5708) (end 132.969 97.3404) (width 0.25) (layer B.Cu) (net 12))
 (segment (start 132.2324 95.8342) (end 132.969 96.5708) (width 0.25) (layer B.Cu) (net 12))
 (segment (start 129.4384 95.8342) (end 132.2324 95.8342) (width 0.25) (layer B.Cu) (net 12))
 (segment (start 128.3462 96.9264) (end 129.4384 95.8342) (width 0.25) (layer B.Cu) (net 12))
 (segment (start 127.8154 117.4242) (end 127.8154 98.524) (width 0.25) (layer F.Cu) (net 12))
 (segment (start 128.3462 97.9932) (end 128.3716 98.0186) (width 0.25) (layer B.Cu) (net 12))
 (via (at 128.3462 97.9932) (size 0.6) (drill 0.4) (layers F.Cu B.Cu) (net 12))
 (segment (start 127.8154 98.524) (end 128.3462 97.9932) (width 0.25) (layer F.Cu) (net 12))
 (segment (start 127.8154 117.2596) (end 127.8154 117.4242) (width 0.1524) (layer F.Cu) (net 12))
 (segment (start 132.969 97.3404) (end 132.969 96.52) (width 0.1524) (layer B.Cu) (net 12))
 (segment (start 134.747 95.9866) (end 135.509 96.7486) (width 0.1524) (layer B.Cu) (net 12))
 (segment (start 133.5024 95.9866) (end 134.747 95.9866) (width 0.1524) (layer B.Cu) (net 12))
 (segment (start 132.969 96.52) (end 133.5024 95.9866) (width 0.1524) (layer B.Cu) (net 12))
 (segment (start 135.509 96.7486) (end 135.509 97.3404) (width 0.1524) (layer B.Cu) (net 12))
 (segment (start 132.0673 84.58708) (end 132.0673 88.9635) (width 0.25) (layer B.Cu) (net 7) (status 400000))
 (segment (start 130.429 90.4367) (end 130.429 91.9404) (width 0.25) (layer B.Cu) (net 7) (status 800000))
 (segment (start 130.9243 89.9414) (end 130.429 90.4367) (width 0.25) (layer B.Cu) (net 7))
 (segment (start 131.0894 89.9414) (end 130.9243 89.9414) (width 0.25) (layer B.Cu) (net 7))
 (segment (start 132.0673 88.9635) (end 131.0894 89.9414) (width 0.25) (layer B.Cu) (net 7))
 (segment (start 133.1976 65.4812) (end 133.1976 66.04) (width 0.5) (layer B.Cu) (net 1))
 (segment (start 133.1976 66.04) (end 128.0668 71.1708) (width 0.5) (layer B.Cu) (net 1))
 (segment (start 133.1976 65.4812) (end 135.7376 65.4812) (width 0.5) (layer B.Cu) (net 1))
 (segment (start 135.7376 65.4812) (end 140.7668 70.5104) (width 0.5) (layer B.Cu) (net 1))
 (segment (start 140.7668 70.5104) (end 140.7668 71.1708) (width 0.25) (layer B.Cu) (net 1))
 (segment (start 125.5776 73.66) (end 128.0668 71.1708) (width 0.5) (layer B.Cu) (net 1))
 (segment (start 128.0668 71.1708) (end 140.7668 71.1708) (width 0.5) (layer B.Cu) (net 1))
 (segment (start 143.51 96.52) (end 143.51 95.885) (width 0.25) (layer F.Cu) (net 17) (status C00000))
 (segment (start 143.51 95.885) (end 140.8938 93.2688) (width 0.25) (layer F.Cu) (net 17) (status 400000))
 (segment (start 136.0551 84.9376) (end 133.9977 84.9376) (width 0.25) (layer B.Cu) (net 17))
 (segment (start 136.0805 84.9122) (end 136.0551 84.9376) (width 0.25) (layer B.Cu) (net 17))
 (via (at 136.0805 84.9122) (size 0.6) (drill 0.4) (layers F.Cu B.Cu) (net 17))
 (segment (start 137.9728 84.9122) (end 136.0805 84.9122) (width 0.25) (layer F.Cu) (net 17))
 (segment (start 140.8938 87.8332) (end 137.9728 84.9122) (width 0.25) (layer F.Cu) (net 17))
 (segment (start 140.8938 93.2688) (end 140.8938 87.8332) (width 0.25) (layer F.Cu) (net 17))
 (segment (start 143.51 96.52) (end 143.51 96.266) (width 0.25) (layer F.Cu) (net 17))
 (segment (start 133.9977 85.60566) (end 133.0173 86.58606) (width 0.25) (layer B.Cu) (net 17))
 (segment (start 132.4665 82.6643) (end 133.5151 82.6643) (width 0.25) (layer B.Cu) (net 17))
 (segment (start 133.9977 83.1469) (end 133.9977 84.1629) (width 0.25) (layer B.Cu) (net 17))
 (segment (start 133.9977 84.1629) (end 133.9977 84.2899) (width 0.25) (layer B.Cu) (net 17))
 (segment (start 133.9977 84.2899) (end 133.9977 84.9376) (width 0.25) (layer B.Cu) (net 17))
 (segment (start 133.9977 84.9376) (end 133.9977 85.60566) (width 0.25) (layer B.Cu) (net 17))
 (segment (start 133.5151 82.6643) (end 133.9977 83.1469) (width 0.25) (layer B.Cu) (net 17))
 (segment (start 136.779 91.9404) (end 136.779 92.6592) (width 0.25) (layer B.Cu) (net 8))
 (segment (start 136.779 92.6592) (end 138.6586 94.5388) (width 0.25) (layer B.Cu) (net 8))
 (segment (start 141.8844 97.4344) (end 143.51 99.06) (width 0.25) (layer B.Cu) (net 8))
 (segment (start 141.8844 95.9358) (end 141.8844 97.4344) (width 0.25) (layer B.Cu) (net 8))
 (segment (start 140.4874 94.5388) (end 141.8844 95.9358) (width 0.25) (layer B.Cu) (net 8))
 (segment (start 138.6586 94.5388) (end 140.4874 94.5388) (width 0.25) (layer B.Cu) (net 8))
 (segment (start 135.509 91.9404) (end 136.779 91.9404) (width 0.25) (layer B.Cu) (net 8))
 (segment (start 140.7922 97.2146) (end 140.9026 97.2146) (width 0.25) (layer B.Cu) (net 11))
 (segment (start 140.9026 97.2146) (end 141.6812 97.9932) (width 0.25) (layer B.Cu) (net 11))
 (segment (start 141.6812 99.8474) (end 143.4338 101.6) (width 0.25) (layer B.Cu) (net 11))
 (segment (start 141.6812 97.9932) (end 141.6812 99.8474) (width 0.25) (layer B.Cu) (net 11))
 (segment (start 143.4338 101.6) (end 143.51 101.6) (width 0.25) (layer B.Cu) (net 11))
 (segment (start 138.049 97.3404) (end 138.049 96.2406) (width 0.25) (layer B.Cu) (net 11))
 (segment (start 140.7922 96.5454) (end 140.7922 97.2146) (width 0.25) (layer B.Cu) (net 11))
 (segment (start 139.9794 95.7326) (end 140.7922 96.5454) (width 0.25) (layer B.Cu) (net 11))
 (segment (start 138.557 95.7326) (end 139.9794 95.7326) (width 0.25) (layer B.Cu) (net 11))
 (segment (start 138.049 96.2406) (end 138.557 95.7326) (width 0.25) (layer B.Cu) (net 11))
 (segment (start 136.779 97.3404) (end 138.049 97.3404) (width 0.25) (layer B.Cu) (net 11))
 (segment (start 125.73 99.06) (end 125.7554 99.06) (width 0.25) (layer B.Cu) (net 19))
 (segment (start 125.7554 99.06) (end 127.508 97.3074) (width 0.25) (layer B.Cu) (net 19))
 (segment (start 127.508 97.3074) (end 127.508 93.16) (width 0.25) (layer B.Cu) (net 19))
 (segment (start 127.508 93.16) (end 128.905 93.16) (width 0.25) (layer B.Cu) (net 19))
 (segment (start 143.51 83.82) (end 136.3726 83.82) (width 0.25) (layer F.Cu) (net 18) (status 400000))
 (segment (start 131.5665 81.603) (end 131.5665 82.6643) (width 0.25) (layer B.Cu) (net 18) (status 800000))
 (segment (start 131.6101 81.5594) (end 131.5665 81.603) (width 0.25) (layer B.Cu) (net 18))
 (via (at 131.6101 81.5594) (size 0.6) (drill 0.4) (layers F.Cu B.Cu) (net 18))
 (segment (start 131.6355 81.534) (end 131.6101 81.5594) (width 0.25) (layer F.Cu) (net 18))
 (segment (start 134.0866 81.534) (end 131.6355 81.534) (width 0.25) (layer F.Cu) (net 18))
 (segment (start 136.3726 83.82) (end 134.0866 81.534) (width 0.25) (layer F.Cu) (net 18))
 (segment (start 131.1173 86.58606) (end 130.83286 86.58606) (width 0.25) (layer B.Cu) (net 18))
 (segment (start 130.83286 86.58606) (end 130.1877 85.9409) (width 0.5) (layer B.Cu) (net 18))
 (segment (start 130.1877 85.9409) (end 130.1877 84.0431) (width 0.5) (layer B.Cu) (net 18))
 (segment (start 130.1877 84.0431) (end 131.5665 82.6643) (width 0.5) (layer B.Cu) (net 18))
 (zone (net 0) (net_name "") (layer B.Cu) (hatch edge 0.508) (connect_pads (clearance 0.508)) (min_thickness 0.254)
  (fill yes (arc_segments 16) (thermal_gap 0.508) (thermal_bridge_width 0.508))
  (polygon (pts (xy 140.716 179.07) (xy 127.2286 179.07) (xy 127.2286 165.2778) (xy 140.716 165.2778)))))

